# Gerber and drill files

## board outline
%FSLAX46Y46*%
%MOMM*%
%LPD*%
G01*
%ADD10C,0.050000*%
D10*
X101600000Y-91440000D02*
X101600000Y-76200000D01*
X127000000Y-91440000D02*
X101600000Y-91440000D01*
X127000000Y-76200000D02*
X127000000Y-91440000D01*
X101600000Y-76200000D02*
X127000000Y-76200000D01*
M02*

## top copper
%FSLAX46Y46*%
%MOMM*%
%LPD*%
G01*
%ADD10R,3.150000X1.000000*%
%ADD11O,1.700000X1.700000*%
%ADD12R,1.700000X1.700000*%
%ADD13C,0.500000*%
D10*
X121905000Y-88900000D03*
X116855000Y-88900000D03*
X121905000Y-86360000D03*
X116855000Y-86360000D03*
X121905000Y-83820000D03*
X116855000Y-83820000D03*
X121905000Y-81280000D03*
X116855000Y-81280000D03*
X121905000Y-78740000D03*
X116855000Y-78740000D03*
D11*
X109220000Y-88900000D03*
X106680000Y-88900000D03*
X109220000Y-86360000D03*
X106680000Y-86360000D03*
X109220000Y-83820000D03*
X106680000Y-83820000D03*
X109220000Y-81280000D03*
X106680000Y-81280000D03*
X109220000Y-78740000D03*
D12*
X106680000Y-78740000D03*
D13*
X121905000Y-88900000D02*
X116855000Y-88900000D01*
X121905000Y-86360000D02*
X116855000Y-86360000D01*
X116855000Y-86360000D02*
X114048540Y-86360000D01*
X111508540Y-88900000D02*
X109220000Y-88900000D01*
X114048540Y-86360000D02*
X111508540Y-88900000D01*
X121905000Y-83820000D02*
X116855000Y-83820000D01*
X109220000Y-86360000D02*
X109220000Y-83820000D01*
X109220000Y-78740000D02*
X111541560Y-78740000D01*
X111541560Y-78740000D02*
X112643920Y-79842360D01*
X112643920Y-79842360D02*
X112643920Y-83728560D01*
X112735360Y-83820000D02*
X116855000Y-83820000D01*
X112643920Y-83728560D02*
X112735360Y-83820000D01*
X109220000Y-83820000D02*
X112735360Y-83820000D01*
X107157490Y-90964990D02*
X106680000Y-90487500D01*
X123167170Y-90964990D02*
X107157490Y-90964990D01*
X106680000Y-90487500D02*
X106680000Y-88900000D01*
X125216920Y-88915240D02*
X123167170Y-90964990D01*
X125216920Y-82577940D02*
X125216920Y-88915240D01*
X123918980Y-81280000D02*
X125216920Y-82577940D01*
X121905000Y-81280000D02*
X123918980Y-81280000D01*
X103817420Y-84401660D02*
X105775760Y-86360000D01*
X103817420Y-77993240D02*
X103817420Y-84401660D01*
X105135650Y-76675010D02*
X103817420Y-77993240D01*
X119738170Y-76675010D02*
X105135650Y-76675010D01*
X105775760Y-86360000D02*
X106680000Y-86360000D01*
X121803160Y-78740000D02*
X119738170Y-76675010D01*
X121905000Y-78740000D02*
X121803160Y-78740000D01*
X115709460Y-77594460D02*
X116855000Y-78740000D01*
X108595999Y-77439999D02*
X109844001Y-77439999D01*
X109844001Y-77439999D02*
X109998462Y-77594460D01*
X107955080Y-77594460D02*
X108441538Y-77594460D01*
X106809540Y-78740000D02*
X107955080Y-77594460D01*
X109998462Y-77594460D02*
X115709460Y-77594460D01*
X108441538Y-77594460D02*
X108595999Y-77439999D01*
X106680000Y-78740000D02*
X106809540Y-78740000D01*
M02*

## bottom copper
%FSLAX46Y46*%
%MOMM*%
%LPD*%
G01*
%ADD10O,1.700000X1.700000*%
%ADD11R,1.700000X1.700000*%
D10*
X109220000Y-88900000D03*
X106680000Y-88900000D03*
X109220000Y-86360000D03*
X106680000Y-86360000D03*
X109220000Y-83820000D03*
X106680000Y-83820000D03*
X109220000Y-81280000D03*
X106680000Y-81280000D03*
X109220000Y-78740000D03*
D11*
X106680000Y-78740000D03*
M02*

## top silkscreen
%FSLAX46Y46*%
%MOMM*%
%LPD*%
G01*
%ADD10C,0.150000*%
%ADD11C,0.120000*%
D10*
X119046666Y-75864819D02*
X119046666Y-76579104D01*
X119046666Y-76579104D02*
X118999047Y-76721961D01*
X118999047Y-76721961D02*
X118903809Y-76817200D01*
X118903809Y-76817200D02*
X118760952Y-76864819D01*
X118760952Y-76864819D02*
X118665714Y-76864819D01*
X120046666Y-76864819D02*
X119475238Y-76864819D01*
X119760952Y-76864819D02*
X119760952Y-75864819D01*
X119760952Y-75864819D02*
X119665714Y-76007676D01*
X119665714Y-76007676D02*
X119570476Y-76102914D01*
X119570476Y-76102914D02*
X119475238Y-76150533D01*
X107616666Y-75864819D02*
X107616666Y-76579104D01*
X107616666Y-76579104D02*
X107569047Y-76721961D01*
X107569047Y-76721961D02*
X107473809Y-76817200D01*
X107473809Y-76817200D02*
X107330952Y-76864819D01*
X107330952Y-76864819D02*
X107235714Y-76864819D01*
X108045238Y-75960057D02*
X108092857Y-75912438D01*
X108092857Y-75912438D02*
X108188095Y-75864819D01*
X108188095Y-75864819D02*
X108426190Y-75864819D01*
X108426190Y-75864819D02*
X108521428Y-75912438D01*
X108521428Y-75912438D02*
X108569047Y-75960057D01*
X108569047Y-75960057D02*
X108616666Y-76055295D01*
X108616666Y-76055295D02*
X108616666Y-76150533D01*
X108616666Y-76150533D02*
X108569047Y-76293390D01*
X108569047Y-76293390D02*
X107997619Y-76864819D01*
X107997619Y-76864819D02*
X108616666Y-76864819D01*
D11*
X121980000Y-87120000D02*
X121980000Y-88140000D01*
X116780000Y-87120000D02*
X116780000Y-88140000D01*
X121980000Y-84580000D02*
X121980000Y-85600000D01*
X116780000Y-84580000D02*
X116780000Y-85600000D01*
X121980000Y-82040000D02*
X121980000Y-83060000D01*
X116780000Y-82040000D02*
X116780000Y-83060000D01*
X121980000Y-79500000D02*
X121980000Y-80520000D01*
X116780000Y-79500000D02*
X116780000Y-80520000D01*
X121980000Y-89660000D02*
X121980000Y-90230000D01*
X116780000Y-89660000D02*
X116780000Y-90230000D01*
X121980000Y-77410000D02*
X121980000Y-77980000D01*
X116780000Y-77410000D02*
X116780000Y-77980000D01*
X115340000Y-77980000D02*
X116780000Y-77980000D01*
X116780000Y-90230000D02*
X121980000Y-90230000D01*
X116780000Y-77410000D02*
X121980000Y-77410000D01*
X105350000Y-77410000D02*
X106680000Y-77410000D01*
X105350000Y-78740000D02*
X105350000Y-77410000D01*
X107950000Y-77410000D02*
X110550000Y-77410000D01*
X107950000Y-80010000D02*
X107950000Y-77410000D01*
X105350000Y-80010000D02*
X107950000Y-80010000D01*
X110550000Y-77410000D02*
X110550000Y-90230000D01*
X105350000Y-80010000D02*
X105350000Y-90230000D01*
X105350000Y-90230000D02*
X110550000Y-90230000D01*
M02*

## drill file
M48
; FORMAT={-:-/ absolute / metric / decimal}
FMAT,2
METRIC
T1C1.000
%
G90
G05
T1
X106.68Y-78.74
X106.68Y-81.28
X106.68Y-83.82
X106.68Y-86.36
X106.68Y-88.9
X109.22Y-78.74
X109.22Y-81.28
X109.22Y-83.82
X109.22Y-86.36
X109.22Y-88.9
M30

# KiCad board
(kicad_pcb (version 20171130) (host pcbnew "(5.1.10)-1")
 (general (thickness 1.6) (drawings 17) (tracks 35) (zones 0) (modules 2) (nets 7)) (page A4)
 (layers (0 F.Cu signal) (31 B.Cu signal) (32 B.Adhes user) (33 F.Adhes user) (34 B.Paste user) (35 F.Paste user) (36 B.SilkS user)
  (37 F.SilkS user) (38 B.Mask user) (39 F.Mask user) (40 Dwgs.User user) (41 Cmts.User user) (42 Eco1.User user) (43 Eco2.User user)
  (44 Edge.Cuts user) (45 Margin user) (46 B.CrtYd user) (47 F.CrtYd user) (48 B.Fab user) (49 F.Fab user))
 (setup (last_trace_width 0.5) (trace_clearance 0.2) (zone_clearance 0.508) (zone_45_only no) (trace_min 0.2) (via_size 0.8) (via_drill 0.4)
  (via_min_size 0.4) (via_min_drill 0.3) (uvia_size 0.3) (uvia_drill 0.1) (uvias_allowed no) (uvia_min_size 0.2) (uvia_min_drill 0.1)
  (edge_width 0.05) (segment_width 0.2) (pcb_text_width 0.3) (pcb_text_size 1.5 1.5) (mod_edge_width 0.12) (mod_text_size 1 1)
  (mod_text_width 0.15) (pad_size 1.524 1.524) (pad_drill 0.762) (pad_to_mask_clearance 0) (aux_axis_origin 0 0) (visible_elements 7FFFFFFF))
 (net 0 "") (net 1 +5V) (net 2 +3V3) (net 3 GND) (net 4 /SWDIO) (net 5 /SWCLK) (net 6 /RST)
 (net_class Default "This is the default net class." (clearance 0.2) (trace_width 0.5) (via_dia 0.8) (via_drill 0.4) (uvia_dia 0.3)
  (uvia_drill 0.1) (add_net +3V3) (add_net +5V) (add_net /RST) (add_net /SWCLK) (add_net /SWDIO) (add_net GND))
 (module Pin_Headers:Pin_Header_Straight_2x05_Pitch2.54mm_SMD (layer F.Cu) (at 119.38 83.82)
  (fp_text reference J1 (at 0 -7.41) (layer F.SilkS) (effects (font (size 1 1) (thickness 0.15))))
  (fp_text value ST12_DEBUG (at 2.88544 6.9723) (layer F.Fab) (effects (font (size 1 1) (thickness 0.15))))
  (fp_line (start 2.6 3.3) (end 2.6 4.32) (layer F.SilkS) (width 0.12))
  (fp_line (start -2.6 3.3) (end -2.6 4.32) (layer F.SilkS) (width 0.12))
  (fp_line (start 2.6 0.76) (end 2.6 1.78) (layer F.SilkS) (width 0.12))
  (fp_line (start -2.6 0.76) (end -2.6 1.78) (layer F.SilkS) (width 0.12))
  (fp_line (start 2.6 -1.78) (end 2.6 -0.76) (layer F.SilkS) (width 0.12))
  (fp_line (start -2.6 -1.78) (end -2.6 -0.76) (layer F.SilkS) (width 0.12))
  (fp_line (start 2.6 -4.32) (end 2.6 -3.3) (layer F.SilkS) (width 0.12))
  (fp_line (start -2.6 -4.32) (end -2.6 -3.3) (layer F.SilkS) (width 0.12))
  (fp_line (start 2.6 5.84) (end 2.6 6.41) (layer F.SilkS) (width 0.12))
  (fp_line (start -2.6 5.84) (end -2.6 6.41) (layer F.SilkS) (width 0.12))
  (fp_line (start 2.6 -6.41) (end 2.6 -5.84) (layer F.SilkS) (width 0.12))
  (fp_line (start -2.6 -6.41) (end -2.6 -5.84) (layer F.SilkS) (width 0.12))
  (fp_line (start -4.04 -5.84) (end -2.6 -5.84) (layer F.SilkS) (width 0.12))
  (fp_line (start -2.6 6.41) (end 2.6 6.41) (layer F.SilkS) (width 0.12))
  (fp_line (start -2.6 -6.41) (end 2.6 -6.41) (layer F.SilkS) (width 0.12))
  (pad 10 smd rect (at 2.525 5.08) (size 3.15 1) (layers F.Cu F.Paste F.Mask) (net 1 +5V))
  (pad 9 smd rect (at -2.525 5.08) (size 3.15 1) (layers F.Cu F.Paste F.Mask) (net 1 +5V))
  (pad 8 smd rect (at 2.525 2.54) (size 3.15 1) (layers F.Cu F.Paste F.Mask) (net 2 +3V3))
  (pad 7 smd rect (at -2.525 2.54) (size 3.15 1) (layers F.Cu F.Paste F.Mask) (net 2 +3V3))
  (pad 6 smd rect (at 2.525 0) (size 3.15 1) (layers F.Cu F.Paste F.Mask) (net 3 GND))
  (pad 5 smd rect (at -2.525 0) (size 3.15 1) (layers F.Cu F.Paste F.Mask) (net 3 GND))
  (pad 4 smd rect (at 2.525 -2.54) (size 3.15 1) (layers F.Cu F.Paste F.Mask) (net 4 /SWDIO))
  (pad 3 smd rect (at -2.525 -2.54) (size 3.15 1) (layers F.Cu F.Paste F.Mask))
  (pad 2 smd rect (at 2.525 -5.08) (size 3.15 1) (layers F.Cu F.Paste F.Mask) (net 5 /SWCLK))
  (pad 1 smd rect (at -2.525 -5.08) (size 3.15 1) (layers F.Cu F.Paste F.Mask) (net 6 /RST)))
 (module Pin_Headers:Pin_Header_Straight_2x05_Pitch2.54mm (layer F.Cu) (at 106.68 78.74)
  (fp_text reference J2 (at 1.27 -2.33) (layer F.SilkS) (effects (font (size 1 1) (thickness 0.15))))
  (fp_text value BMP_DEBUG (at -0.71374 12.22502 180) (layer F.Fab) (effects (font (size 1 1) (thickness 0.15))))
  (fp_line (start -1.33 -1.33) (end 0 -1.33) (layer F.SilkS) (width 0.12))
  (fp_line (start -1.33 0) (end -1.33 -1.33) (layer F.SilkS) (width 0.12))
  (fp_line (start 1.27 -1.33) (end 3.87 -1.33) (layer F.SilkS) (width 0.12))
  (fp_line (start 1.27 1.27) (end 1.27 -1.33) (layer F.SilkS) (width 0.12))
  (fp_line (start -1.33 1.27) (end 1.27 1.27) (layer F.SilkS) (width 0.12))
  (fp_line (start 3.87 -1.33) (end 3.87 11.49) (layer F.SilkS) (width 0.12))
  (fp_line (start -1.33 1.27) (end -1.33 11.49) (layer F.SilkS) (width 0.12))
  (fp_line (start -1.33 11.49) (end 3.87 11.49) (layer F.SilkS) (width 0.12))
  (pad 10 thru_hole oval (at 2.54 10.16) (size 1.7 1.7) (drill 1) (layers *.Cu *.Mask) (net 2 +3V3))
  (pad 9 thru_hole oval (at 0 10.16) (size 1.7 1.7) (drill 1) (layers *.Cu *.Mask) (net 4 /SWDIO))
  (pad 8 thru_hole oval (at 2.54 7.62) (size 1.7 1.7) (drill 1) (layers *.Cu *.Mask) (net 3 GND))
  (pad 7 thru_hole oval (at 0 7.62) (size 1.7 1.7) (drill 1) (layers *.Cu *.Mask) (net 5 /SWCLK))
  (pad 6 thru_hole oval (at 2.54 5.08) (size 1.7 1.7) (drill 1) (layers *.Cu *.Mask) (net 3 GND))
  (pad 5 thru_hole oval (at 0 5.08) (size 1.7 1.7) (drill 1) (layers *.Cu *.Mask))
  (pad 4 thru_hole oval (at 2.54 2.54) (size 1.7 1.7) (drill 1) (layers *.Cu *.Mask))
  (pad 3 thru_hole oval (at 0 2.54) (size 1.7 1.7) (drill 1) (layers *.Cu *.Mask))
  (pad 2 thru_hole oval (at 2.54 0) (size 1.7 1.7) (drill 1) (layers *.Cu *.Mask) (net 3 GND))
  (pad 1 thru_hole rect (at 0 0) (size 1.7 1.7) (drill 1) (layers *.Cu *.Mask) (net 6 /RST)))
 (gr_line (start 101.6 91.44) (end 101.6 76.2) (layer Edge.Cuts) (width 0.05))
 (gr_line (start 127 91.44) (end 101.6 91.44) (layer Edge.Cuts) (width 0.05))
 (gr_line (start 127 76.2) (end 127 91.44) (layer Edge.Cuts) (width 0.05))
 (gr_line (start 101.6 76.2) (end 127 76.2) (layer Edge.Cuts) (width 0.05))
 (segment (start 121.905 88.9) (end 116.855 88.9) (width 0.5) (layer F.Cu) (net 1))
 (segment (start 121.905 86.36) (end 116.855 86.36) (width 0.5) (layer F.Cu) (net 2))
 (segment (start 116.855 86.36) (end 114.04854 86.36) (width 0.5) (layer F.Cu) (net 2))
 (segment (start 111.50854 88.9) (end 109.22 88.9) (width 0.5) (layer F.Cu) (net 2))
 (segment (start 114.04854 86.36) (end 111.50854 88.9) (width 0.5) (layer F.Cu) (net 2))
 (segment (start 121.905 83.82) (end 116.855 83.82) (width 0.5) (layer F.Cu) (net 3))
 (segment (start 109.22 86.36) (end 109.22 83.82) (width 0.5) (layer F.Cu) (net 3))
 (segment (start 109.22 78.74) (end 111.54156 78.74) (width 0.5) (layer F.Cu) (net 3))
 (segment (start 111.54156 78.74) (end 112.64392 79.84236) (width 0.5) (layer F.Cu) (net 3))
 (segment (start 112.64392 79.84236) (end 112.64392 83.72856) (width 0.5) (layer F.Cu) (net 3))
 (segment (start 112.73536 83.82) (end 116.855 83.82) (width 0.5) (layer F.Cu) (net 3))
 (segment (start 112.64392 83.72856) (end 112.73536 83.82) (width 0.5) (layer F.Cu) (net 3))
 (segment (start 109.22 83.82) (end 112.73536 83.82) (width 0.5) (layer F.Cu) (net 3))
 (segment (start 107.15749 90.96499) (end 106.68 90.4875) (width 0.5) (layer F.Cu) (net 4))
 (segment (start 123.16717 90.96499) (end 107.15749 90.96499) (width 0.5) (layer F.Cu) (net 4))
 (segment (start 106.68 90.4875) (end 106.68 88.9) (width 0.5) (layer F.Cu) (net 4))
 (segment (start 125.21692 88.91524) (end 123.16717 90.96499) (width 0.5) (layer F.Cu) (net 4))
 (segment (start 125.21692 82.57794) (end 125.21692 88.91524) (width 0.5) (layer F.Cu) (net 4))
 (segment (start 123.91898 81.28) (end 125.21692 82.57794) (width 0.5) (layer F.Cu) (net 4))
 (segment (start 121.905 81.28) (end 123.91898 81.28) (width 0.5) (layer F.Cu) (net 4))
 (segment (start 103.81742 84.40166) (end 105.77576 86.36) (width 0.5) (layer F.Cu) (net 5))
 (segment (start 103.81742 77.99324) (end 103.81742 84.40166) (width 0.5) (layer F.Cu) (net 5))
 (segment (start 105.13565 76.67501) (end 103.81742 77.99324) (width 0.5) (layer F.Cu) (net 5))
 (segment (start 119.73817 76.67501) (end 105.13565 76.67501) (width 0.5) (layer F.Cu) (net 5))
 (segment (start 105.77576 86.36) (end 106.68 86.36) (width 0.5) (layer F.Cu) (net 5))
 (segment (start 121.80316 78.74) (end 119.73817 76.67501) (width 0.5) (layer F.Cu) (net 5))
 (segment (start 121.905 78.74) (end 121.80316 78.74) (width 0.5) (layer F.Cu) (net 5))
 (segment (start 115.70946 77.59446) (end 116.855 78.74) (width 0.5) (layer F.Cu) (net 6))
 (segment (start 108.595999 77.439999) (end 109.844001 77.439999) (width 0.5) (layer F.Cu) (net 6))
 (segment (start 109.844001 77.439999) (end 109.998462 77.59446) (width 0.5) (layer F.Cu) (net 6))
 (segment (start 107.95508 77.59446) (end 108.441538 77.59446) (width 0.5) (layer F.Cu) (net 6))
 (segment (start 106.80954 78.74) (end 107.95508 77.59446) (width 0.5) (layer F.Cu) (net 6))
 (segment (start 109.998462 77.59446) (end 115.70946 77.59446) (width 0.5) (layer F.Cu) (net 6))
 (segment (start 108.441538 77.59446) (end 108.595999 77.439999) (width 0.5) (layer F.Cu) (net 6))
 (segment (start 106.68 78.74) (end 106.80954 78.74) (width 0.5) (layer F.Cu) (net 6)))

